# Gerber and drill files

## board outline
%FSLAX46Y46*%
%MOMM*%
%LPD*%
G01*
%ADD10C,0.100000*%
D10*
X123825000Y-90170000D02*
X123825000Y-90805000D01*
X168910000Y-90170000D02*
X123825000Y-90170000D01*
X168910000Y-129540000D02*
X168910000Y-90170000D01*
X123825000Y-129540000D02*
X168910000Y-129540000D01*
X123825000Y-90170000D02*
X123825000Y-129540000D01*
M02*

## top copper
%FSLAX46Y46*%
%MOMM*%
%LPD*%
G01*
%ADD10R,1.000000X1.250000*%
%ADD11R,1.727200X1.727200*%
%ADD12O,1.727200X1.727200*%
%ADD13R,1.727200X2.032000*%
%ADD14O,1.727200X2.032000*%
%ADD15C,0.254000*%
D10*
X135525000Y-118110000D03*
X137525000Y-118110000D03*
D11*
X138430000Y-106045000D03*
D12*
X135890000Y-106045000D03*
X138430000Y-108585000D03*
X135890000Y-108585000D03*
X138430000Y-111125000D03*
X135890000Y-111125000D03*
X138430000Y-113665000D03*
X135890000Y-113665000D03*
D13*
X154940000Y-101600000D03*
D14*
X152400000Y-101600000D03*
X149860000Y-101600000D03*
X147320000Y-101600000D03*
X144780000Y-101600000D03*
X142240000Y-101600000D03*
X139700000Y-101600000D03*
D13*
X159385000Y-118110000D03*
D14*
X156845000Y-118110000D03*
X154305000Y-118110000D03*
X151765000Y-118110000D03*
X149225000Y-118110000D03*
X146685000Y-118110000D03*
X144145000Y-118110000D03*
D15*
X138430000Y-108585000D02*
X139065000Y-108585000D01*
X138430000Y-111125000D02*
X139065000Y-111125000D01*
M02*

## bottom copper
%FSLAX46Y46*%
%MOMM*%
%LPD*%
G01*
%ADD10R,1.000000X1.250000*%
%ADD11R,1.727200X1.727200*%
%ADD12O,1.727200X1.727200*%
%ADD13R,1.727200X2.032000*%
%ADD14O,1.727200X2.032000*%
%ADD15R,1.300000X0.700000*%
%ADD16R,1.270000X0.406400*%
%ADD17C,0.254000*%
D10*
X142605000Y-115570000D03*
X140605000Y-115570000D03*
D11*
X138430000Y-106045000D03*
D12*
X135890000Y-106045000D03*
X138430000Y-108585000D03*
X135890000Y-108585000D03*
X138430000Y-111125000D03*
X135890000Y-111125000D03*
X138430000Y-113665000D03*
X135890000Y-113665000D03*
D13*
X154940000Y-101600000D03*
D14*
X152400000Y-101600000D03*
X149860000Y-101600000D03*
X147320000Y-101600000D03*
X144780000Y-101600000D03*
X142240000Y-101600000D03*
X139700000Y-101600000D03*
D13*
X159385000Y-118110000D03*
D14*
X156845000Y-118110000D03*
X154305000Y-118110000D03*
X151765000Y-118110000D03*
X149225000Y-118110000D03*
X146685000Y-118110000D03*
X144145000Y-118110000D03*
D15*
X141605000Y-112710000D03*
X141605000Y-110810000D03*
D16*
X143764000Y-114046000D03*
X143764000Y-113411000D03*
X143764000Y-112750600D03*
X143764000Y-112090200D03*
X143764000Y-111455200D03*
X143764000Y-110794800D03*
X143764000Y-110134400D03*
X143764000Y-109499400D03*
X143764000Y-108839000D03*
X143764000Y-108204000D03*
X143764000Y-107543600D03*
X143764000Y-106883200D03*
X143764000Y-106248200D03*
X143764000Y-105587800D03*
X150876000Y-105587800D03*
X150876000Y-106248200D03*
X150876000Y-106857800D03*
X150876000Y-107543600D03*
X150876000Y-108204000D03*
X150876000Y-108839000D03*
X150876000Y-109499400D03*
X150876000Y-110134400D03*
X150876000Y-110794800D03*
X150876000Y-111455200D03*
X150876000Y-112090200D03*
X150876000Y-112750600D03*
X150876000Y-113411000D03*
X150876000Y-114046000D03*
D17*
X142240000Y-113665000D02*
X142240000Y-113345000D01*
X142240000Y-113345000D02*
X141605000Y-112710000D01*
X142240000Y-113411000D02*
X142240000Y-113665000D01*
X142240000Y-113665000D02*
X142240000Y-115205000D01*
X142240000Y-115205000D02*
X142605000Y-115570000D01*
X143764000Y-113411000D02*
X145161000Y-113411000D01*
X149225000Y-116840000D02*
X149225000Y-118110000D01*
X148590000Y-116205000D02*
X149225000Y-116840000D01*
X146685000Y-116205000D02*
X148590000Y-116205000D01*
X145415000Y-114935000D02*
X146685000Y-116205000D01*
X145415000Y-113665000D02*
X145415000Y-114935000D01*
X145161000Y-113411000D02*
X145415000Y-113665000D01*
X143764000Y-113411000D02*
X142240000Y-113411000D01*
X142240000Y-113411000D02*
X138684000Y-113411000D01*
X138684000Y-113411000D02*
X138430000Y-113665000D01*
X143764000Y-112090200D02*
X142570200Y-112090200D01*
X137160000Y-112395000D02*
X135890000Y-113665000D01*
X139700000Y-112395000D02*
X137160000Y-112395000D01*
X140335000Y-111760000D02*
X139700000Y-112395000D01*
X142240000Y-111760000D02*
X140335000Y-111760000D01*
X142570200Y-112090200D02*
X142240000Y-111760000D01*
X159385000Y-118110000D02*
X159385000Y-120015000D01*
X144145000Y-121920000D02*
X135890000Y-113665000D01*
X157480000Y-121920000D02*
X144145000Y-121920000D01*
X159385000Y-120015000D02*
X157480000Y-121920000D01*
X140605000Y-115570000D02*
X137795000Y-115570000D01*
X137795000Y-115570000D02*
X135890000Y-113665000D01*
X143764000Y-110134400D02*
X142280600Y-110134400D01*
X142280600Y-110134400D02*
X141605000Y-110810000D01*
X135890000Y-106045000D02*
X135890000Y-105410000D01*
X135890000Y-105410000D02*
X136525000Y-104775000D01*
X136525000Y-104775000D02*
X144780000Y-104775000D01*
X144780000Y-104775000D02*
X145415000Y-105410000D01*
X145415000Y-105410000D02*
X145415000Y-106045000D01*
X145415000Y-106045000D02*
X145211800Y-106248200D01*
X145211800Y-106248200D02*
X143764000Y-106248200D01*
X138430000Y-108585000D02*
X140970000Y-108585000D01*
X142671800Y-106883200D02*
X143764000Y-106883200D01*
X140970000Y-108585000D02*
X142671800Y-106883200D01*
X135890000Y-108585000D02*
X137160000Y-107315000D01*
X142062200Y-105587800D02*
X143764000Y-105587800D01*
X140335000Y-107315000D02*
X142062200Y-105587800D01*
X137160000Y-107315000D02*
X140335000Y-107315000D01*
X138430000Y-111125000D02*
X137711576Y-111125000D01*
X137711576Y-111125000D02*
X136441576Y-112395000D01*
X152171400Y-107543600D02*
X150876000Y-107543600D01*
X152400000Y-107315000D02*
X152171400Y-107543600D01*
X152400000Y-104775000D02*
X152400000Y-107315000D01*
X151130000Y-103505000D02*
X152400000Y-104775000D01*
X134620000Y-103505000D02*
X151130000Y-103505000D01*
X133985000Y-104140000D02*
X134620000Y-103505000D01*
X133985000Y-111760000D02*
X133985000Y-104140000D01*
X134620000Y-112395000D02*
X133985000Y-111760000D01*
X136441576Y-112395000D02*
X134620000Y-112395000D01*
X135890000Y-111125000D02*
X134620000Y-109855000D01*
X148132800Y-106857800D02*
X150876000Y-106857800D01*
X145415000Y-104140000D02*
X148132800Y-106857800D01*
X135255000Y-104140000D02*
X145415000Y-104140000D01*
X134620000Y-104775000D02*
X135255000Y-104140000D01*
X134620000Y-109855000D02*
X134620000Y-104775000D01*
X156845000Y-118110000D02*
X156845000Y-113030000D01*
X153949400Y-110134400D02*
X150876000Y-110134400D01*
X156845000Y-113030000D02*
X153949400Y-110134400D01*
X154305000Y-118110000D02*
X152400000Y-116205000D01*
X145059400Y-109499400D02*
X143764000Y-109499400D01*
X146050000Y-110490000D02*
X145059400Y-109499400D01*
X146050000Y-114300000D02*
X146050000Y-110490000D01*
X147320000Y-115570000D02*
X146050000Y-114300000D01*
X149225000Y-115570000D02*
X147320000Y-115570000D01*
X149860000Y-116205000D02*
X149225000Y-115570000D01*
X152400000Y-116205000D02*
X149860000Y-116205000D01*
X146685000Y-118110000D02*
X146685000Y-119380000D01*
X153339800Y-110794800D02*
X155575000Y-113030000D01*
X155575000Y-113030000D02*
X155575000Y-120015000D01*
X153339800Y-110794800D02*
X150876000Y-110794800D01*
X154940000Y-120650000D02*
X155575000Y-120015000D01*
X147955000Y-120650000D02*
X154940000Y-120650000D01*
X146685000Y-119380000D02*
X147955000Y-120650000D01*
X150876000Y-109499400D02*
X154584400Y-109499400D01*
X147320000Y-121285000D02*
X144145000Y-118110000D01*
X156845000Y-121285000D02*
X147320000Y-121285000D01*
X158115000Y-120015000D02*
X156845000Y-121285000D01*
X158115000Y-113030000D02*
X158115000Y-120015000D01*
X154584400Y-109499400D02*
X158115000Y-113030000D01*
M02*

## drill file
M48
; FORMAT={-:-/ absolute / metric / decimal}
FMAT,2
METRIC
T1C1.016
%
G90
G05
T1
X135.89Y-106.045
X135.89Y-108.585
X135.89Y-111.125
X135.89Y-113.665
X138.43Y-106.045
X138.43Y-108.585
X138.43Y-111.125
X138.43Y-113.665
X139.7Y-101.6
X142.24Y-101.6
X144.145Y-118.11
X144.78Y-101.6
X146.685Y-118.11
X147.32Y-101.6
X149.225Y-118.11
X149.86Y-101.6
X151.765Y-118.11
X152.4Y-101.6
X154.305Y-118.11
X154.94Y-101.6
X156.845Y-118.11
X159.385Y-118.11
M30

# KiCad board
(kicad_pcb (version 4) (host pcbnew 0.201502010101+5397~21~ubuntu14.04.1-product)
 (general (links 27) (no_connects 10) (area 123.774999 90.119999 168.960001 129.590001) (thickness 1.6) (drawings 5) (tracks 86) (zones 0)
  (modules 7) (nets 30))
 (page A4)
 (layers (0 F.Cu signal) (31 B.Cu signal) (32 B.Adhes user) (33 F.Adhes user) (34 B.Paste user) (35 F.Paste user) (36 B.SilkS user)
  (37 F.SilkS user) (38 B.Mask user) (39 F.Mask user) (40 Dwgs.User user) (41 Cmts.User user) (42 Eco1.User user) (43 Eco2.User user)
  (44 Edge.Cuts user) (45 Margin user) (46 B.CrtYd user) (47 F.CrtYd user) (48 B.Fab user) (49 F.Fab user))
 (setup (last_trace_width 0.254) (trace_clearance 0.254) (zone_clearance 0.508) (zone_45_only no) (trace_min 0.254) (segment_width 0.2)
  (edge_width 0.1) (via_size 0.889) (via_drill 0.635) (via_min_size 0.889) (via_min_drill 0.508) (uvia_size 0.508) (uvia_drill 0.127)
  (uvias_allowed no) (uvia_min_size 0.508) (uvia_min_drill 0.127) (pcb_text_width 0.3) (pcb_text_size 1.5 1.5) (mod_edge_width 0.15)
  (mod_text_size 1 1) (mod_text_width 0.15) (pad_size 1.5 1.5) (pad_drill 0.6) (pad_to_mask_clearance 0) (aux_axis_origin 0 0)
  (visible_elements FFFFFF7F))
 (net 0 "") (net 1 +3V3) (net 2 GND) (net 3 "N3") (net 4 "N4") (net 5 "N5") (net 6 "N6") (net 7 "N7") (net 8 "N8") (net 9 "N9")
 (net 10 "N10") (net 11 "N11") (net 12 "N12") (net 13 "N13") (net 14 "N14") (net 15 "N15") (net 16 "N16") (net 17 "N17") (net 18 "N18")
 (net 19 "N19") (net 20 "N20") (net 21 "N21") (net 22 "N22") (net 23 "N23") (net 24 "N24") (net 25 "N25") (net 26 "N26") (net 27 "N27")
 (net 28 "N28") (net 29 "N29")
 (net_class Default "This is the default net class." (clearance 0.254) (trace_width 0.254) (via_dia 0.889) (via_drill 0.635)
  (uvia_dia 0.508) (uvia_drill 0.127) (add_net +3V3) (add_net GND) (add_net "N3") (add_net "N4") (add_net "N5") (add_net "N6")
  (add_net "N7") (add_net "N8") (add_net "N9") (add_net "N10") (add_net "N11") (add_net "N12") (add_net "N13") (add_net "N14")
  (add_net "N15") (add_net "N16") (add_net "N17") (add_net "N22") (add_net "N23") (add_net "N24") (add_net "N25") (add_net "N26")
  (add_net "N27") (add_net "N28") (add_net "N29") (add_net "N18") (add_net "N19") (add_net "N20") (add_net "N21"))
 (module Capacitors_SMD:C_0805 (layer B.Cu) (at 141.605 115.57 180)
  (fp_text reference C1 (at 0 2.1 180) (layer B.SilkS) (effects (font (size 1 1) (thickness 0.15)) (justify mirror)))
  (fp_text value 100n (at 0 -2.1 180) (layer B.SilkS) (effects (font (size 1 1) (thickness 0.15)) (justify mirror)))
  (pad 1 smd rect (at -1 0 180) (size 1 1.25) (layers B.Cu B.Paste B.Mask) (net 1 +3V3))
  (pad 2 smd rect (at 1 0 180) (size 1 1.25) (layers B.Cu B.Paste B.Mask) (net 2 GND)))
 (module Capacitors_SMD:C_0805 (layer F.Cu) (at 136.525 118.11)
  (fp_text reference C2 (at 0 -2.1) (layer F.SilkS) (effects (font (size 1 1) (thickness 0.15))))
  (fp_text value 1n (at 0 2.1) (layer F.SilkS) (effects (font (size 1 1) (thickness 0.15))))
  (pad 1 smd rect (at -1 0) (size 1 1.25) (layers F.Cu F.Paste F.Mask) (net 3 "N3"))
  (pad 2 smd rect (at 1 0) (size 1 1.25) (layers F.Cu F.Paste F.Mask) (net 2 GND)))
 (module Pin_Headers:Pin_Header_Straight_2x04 (layer B.Cu) (at 137.16 109.855 270)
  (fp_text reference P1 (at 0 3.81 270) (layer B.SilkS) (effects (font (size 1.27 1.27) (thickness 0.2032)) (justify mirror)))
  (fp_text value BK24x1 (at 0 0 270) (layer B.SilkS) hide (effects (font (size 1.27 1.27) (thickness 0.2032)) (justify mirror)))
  (pad 1 thru_hole rect (at -3.81 -1.27 270) (size 1.7272 1.7272) (drill 1.016) (layers *.Cu *.Mask B.SilkS) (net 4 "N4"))
  (pad 2 thru_hole oval (at -3.81 1.27 270) (size 1.7272 1.7272) (drill 1.016) (layers *.Cu *.Mask B.SilkS) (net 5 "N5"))
  (pad 3 thru_hole oval (at -1.27 -1.27 270) (size 1.7272 1.7272) (drill 1.016) (layers *.Cu *.Mask B.SilkS) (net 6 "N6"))
  (pad 4 thru_hole oval (at -1.27 1.27 270) (size 1.7272 1.7272) (drill 1.016) (layers *.Cu *.Mask B.SilkS) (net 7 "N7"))
  (pad 5 thru_hole oval (at 1.27 -1.27 270) (size 1.7272 1.7272) (drill 1.016) (layers *.Cu *.Mask B.SilkS) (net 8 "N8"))
  (pad 6 thru_hole oval (at 1.27 1.27 270) (size 1.7272 1.7272) (drill 1.016) (layers *.Cu *.Mask B.SilkS) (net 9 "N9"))
  (pad 7 thru_hole oval (at 3.81 -1.27 270) (size 1.7272 1.7272) (drill 1.016) (layers *.Cu *.Mask B.SilkS) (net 1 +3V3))
  (pad 8 thru_hole oval (at 3.81 1.27 270) (size 1.7272 1.7272) (drill 1.016) (layers *.Cu *.Mask B.SilkS) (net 2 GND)))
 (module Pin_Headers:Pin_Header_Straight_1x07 (layer B.Cu) (at 147.32 101.6 180)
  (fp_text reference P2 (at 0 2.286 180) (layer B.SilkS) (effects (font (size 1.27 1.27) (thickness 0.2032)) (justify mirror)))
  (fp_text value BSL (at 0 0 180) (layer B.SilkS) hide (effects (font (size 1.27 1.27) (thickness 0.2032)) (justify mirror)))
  (pad 1 thru_hole rect (at -7.62 0 180) (size 1.7272 2.032) (drill 1.016) (layers *.Cu *.Mask B.SilkS) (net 1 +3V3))
  (pad 2 thru_hole oval (at -5.08 0 180) (size 1.7272 2.032) (drill 1.016) (layers *.Cu *.Mask B.SilkS) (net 2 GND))
  (pad 3 thru_hole oval (at -2.54 0 180) (size 1.7272 2.032) (drill 1.016) (layers *.Cu *.Mask B.SilkS) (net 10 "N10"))
  (pad 4 thru_hole oval (at 0 0 180) (size 1.7272 2.032) (drill 1.016) (layers *.Cu *.Mask B.SilkS) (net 3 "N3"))
  (pad 5 thru_hole oval (at 2.54 0 180) (size 1.7272 2.032) (drill 1.016) (layers *.Cu *.Mask B.SilkS) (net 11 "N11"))
  (pad 6 thru_hole oval (at 5.08 0 180) (size 1.7272 2.032) (drill 1.016) (layers *.Cu *.Mask B.SilkS) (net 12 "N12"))
  (pad 7 thru_hole oval (at 7.62 0 180) (size 1.7272 2.032) (drill 1.016) (layers *.Cu *.Mask B.SilkS) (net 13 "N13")))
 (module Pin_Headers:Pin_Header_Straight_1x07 (layer B.Cu) (at 151.765 118.11 180)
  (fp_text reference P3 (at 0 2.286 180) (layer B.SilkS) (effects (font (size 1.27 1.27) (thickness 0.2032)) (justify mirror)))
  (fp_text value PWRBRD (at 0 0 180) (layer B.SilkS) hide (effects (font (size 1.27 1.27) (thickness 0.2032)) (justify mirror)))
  (pad 1 thru_hole rect (at -7.62 0 180) (size 1.7272 2.032) (drill 1.016) (layers *.Cu *.Mask B.SilkS) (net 2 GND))
  (pad 2 thru_hole oval (at -5.08 0 180) (size 1.7272 2.032) (drill 1.016) (layers *.Cu *.Mask B.SilkS) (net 11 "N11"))
  (pad 3 thru_hole oval (at -2.54 0 180) (size 1.7272 2.032) (drill 1.016) (layers *.Cu *.Mask B.SilkS) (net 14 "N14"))
  (pad 4 thru_hole oval (at 0 0 180) (size 1.7272 2.032) (drill 1.016) (layers *.Cu *.Mask B.SilkS) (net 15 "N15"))
  (pad 5 thru_hole oval (at 2.54 0 180) (size 1.7272 2.032) (drill 1.016) (layers *.Cu *.Mask B.SilkS) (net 1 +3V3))
  (pad 6 thru_hole oval (at 5.08 0 180) (size 1.7272 2.032) (drill 1.016) (layers *.Cu *.Mask B.SilkS) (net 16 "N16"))
  (pad 7 thru_hole oval (at 7.62 0 180) (size 1.7272 2.032) (drill 1.016) (layers *.Cu *.Mask B.SilkS) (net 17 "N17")))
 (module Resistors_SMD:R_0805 (layer B.Cu) (at 141.605 111.76 90)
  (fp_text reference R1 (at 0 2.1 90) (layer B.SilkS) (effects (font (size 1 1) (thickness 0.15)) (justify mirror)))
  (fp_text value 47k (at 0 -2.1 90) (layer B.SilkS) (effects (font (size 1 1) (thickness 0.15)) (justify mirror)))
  (pad 1 smd rect (at -0.95 0 90) (size 0.7 1.3) (layers B.Cu B.Paste B.Mask) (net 1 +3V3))
  (pad 2 smd rect (at 0.95 0 90) (size 0.7 1.3) (layers B.Cu B.Paste B.Mask) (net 3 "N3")))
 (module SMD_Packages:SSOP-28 (layer B.Cu) (at 147.32 109.855 90)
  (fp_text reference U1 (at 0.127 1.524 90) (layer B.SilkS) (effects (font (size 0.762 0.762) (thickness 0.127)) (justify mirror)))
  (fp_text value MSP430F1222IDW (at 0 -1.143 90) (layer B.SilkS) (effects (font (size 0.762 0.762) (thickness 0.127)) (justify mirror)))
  (pad 1 smd rect (at -4.191 -3.556 90) (size 0.4064 1.27) (layers B.Cu B.Paste B.Mask) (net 10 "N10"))
  (pad 2 smd rect (at -3.556 -3.556 90) (size 0.4064 1.27) (layers B.Cu B.Paste B.Mask) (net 1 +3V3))
  (pad 3 smd rect (at -2.8956 -3.556 90) (size 0.4064 1.27) (layers B.Cu B.Paste B.Mask) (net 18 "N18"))
  (pad 4 smd rect (at -2.2352 -3.556 90) (size 0.4064 1.27) (layers B.Cu B.Paste B.Mask) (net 2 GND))
  (pad 5 smd rect (at -1.6002 -3.556 90) (size 0.4064 1.27) (layers B.Cu B.Paste B.Mask) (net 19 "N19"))
  (pad 6 smd rect (at -0.9398 -3.556 90) (size 0.4064 1.27) (layers B.Cu B.Paste B.Mask) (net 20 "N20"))
  (pad 7 smd rect (at -0.2794 -3.556 90) (size 0.4064 1.27) (layers B.Cu B.Paste B.Mask) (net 3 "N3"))
  (pad 8 smd rect (at 0.3556 -3.556 90) (size 0.4064 1.27) (layers B.Cu B.Paste B.Mask) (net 14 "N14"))
  (pad 9 smd rect (at 1.016 -3.556 90) (size 0.4064 1.27) (layers B.Cu B.Paste B.Mask) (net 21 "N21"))
  (pad 10 smd rect (at 1.651 -3.556 90) (size 0.4064 1.27) (layers B.Cu B.Paste B.Mask) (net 12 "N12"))
  (pad 11 smd rect (at 2.3114 -3.556 90) (size 0.4064 1.27) (layers B.Cu B.Paste B.Mask) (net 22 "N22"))
  (pad 12 smd rect (at 2.9718 -3.556 90) (size 0.4064 1.27) (layers B.Cu B.Paste B.Mask) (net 6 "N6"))
  (pad 13 smd rect (at 3.6068 -3.556 90) (size 0.4064 1.27) (layers B.Cu B.Paste B.Mask) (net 5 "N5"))
  (pad 14 smd rect (at 4.2672 -3.556 90) (size 0.4064 1.27) (layers B.Cu B.Paste B.Mask) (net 7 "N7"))
  (pad 15 smd rect (at 4.2672 3.556 90) (size 0.4064 1.27) (layers B.Cu B.Paste B.Mask) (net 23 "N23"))
  (pad 16 smd rect (at 3.6068 3.556 90) (size 0.4064 1.27) (layers B.Cu B.Paste B.Mask) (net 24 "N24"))
  (pad 17 smd rect (at 2.9972 3.556 90) (size 0.4064 1.27) (layers B.Cu B.Paste B.Mask) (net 9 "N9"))
  (pad 18 smd rect (at 2.3114 3.556 90) (size 0.4064 1.27) (layers B.Cu B.Paste B.Mask) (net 8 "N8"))
  (pad 19 smd rect (at 1.651 3.556 90) (size 0.4064 1.27) (layers B.Cu B.Paste B.Mask) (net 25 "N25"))
  (pad 20 smd rect (at 1.016 3.556 90) (size 0.4064 1.27) (layers B.Cu B.Paste B.Mask) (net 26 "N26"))
  (pad 21 smd rect (at 0.3556 3.556 90) (size 0.4064 1.27) (layers B.Cu B.Paste B.Mask) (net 17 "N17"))
  (pad 22 smd rect (at -0.2794 3.556 90) (size 0.4064 1.27) (layers B.Cu B.Paste B.Mask) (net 11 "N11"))
  (pad 23 smd rect (at -0.9398 3.556 90) (size 0.4064 1.27) (layers B.Cu B.Paste B.Mask) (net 16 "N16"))
  (pad 24 smd rect (at -1.6002 3.556 90) (size 0.4064 1.27) (layers B.Cu B.Paste B.Mask) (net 15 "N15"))
  (pad 25 smd rect (at -2.2352 3.556 90) (size 0.4064 1.27) (layers B.Cu B.Paste B.Mask) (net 13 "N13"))
  (pad 26 smd rect (at -2.8956 3.556 90) (size 0.4064 1.27) (layers B.Cu B.Paste B.Mask) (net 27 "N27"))
  (pad 27 smd rect (at -3.556 3.556 90) (size 0.4064 1.27) (layers B.Cu B.Paste B.Mask) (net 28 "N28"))
  (pad 28 smd rect (at -4.191 3.556 90) (size 0.4064 1.27) (layers B.Cu B.Paste B.Mask) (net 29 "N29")))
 (gr_line (start 123.825 90.17) (end 123.825 90.805) (angle 90) (layer Edge.Cuts) (width 0.1))
 (gr_line (start 168.91 90.17) (end 123.825 90.17) (angle 90) (layer Edge.Cuts) (width 0.1))
 (gr_line (start 168.91 129.54) (end 168.91 90.17) (angle 90) (layer Edge.Cuts) (width 0.1))
 (gr_line (start 123.825 129.54) (end 168.91 129.54) (angle 90) (layer Edge.Cuts) (width 0.1))
 (gr_line (start 123.825 90.17) (end 123.825 129.54) (angle 90) (layer Edge.Cuts) (width 0.1))
 (segment (start 142.24 113.665) (end 142.24 113.345) (width 0.254) (layer B.Cu) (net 1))
 (segment (start 142.24 113.345) (end 141.605 112.71) (width 0.254) (layer B.Cu) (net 1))
 (segment (start 142.24 113.411) (end 142.24 113.665) (width 0.254) (layer B.Cu) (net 1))
 (segment (start 142.24 113.665) (end 142.24 115.205) (width 0.254) (layer B.Cu) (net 1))
 (segment (start 142.24 115.205) (end 142.605 115.57) (width 0.254) (layer B.Cu) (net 1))
 (segment (start 143.764 113.411) (end 145.161 113.411) (width 0.254) (layer B.Cu) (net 1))
 (segment (start 149.225 116.84) (end 149.225 118.11) (width 0.254) (layer B.Cu) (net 1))
 (segment (start 148.59 116.205) (end 149.225 116.84) (width 0.254) (layer B.Cu) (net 1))
 (segment (start 146.685 116.205) (end 148.59 116.205) (width 0.254) (layer B.Cu) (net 1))
 (segment (start 145.415 114.935) (end 146.685 116.205) (width 0.254) (layer B.Cu) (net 1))
 (segment (start 145.415 113.665) (end 145.415 114.935) (width 0.254) (layer B.Cu) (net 1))
 (segment (start 145.161 113.411) (end 145.415 113.665) (width 0.254) (layer B.Cu) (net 1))
 (segment (start 143.764 113.411) (end 142.24 113.411) (width 0.254) (layer B.Cu) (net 1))
 (segment (start 142.24 113.411) (end 138.684 113.411) (width 0.254) (layer B.Cu) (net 1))
 (segment (start 138.684 113.411) (end 138.43 113.665) (width 0.254) (layer B.Cu) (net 1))
 (segment (start 143.764 112.0902) (end 142.5702 112.0902) (width 0.254) (layer B.Cu) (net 2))
 (segment (start 137.16 112.395) (end 135.89 113.665) (width 0.254) (layer B.Cu) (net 2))
 (segment (start 139.7 112.395) (end 137.16 112.395) (width 0.254) (layer B.Cu) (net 2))
 (segment (start 140.335 111.76) (end 139.7 112.395) (width 0.254) (layer B.Cu) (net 2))
 (segment (start 142.24 111.76) (end 140.335 111.76) (width 0.254) (layer B.Cu) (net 2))
 (segment (start 142.5702 112.0902) (end 142.24 111.76) (width 0.254) (layer B.Cu) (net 2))
 (segment (start 159.385 118.11) (end 159.385 120.015) (width 0.254) (layer B.Cu) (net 2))
 (segment (start 144.145 121.92) (end 135.89 113.665) (width 0.254) (layer B.Cu) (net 2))
 (segment (start 157.48 121.92) (end 144.145 121.92) (width 0.254) (layer B.Cu) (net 2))
 (segment (start 159.385 120.015) (end 157.48 121.92) (width 0.254) (layer B.Cu) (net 2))
 (segment (start 140.605 115.57) (end 137.795 115.57) (width 0.254) (layer B.Cu) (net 2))
 (segment (start 137.795 115.57) (end 135.89 113.665) (width 0.254) (layer B.Cu) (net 2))
 (segment (start 143.764 110.1344) (end 142.2806 110.1344) (width 0.254) (layer B.Cu) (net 3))
 (segment (start 142.2806 110.1344) (end 141.605 110.81) (width 0.254) (layer B.Cu) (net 3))
 (segment (start 135.89 106.045) (end 135.89 105.41) (width 0.254) (layer B.Cu) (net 5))
 (segment (start 135.89 105.41) (end 136.525 104.775) (width 0.254) (layer B.Cu) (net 5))
 (segment (start 136.525 104.775) (end 144.78 104.775) (width 0.254) (layer B.Cu) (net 5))
 (segment (start 144.78 104.775) (end 145.415 105.41) (width 0.254) (layer B.Cu) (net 5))
 (segment (start 145.415 105.41) (end 145.415 106.045) (width 0.254) (layer B.Cu) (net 5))
 (segment (start 145.415 106.045) (end 145.2118 106.2482) (width 0.254) (layer B.Cu) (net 5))
 (segment (start 145.2118 106.2482) (end 143.764 106.2482) (width 0.254) (layer B.Cu) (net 5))
 (segment (start 138.43 108.585) (end 140.97 108.585) (width 0.254) (layer B.Cu) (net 6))
 (segment (start 142.6718 106.8832) (end 143.764 106.8832) (width 0.254) (layer B.Cu) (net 6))
 (segment (start 140.97 108.585) (end 142.6718 106.8832) (width 0.254) (layer B.Cu) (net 6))
 (segment (start 138.43 108.585) (end 139.065 108.585) (width 0.254) (layer F.Cu) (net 6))
 (segment (start 135.89 108.585) (end 137.16 107.315) (width 0.254) (layer B.Cu) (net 7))
 (segment (start 142.0622 105.5878) (end 143.764 105.5878) (width 0.254) (layer B.Cu) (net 7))
 (segment (start 140.335 107.315) (end 142.0622 105.5878) (width 0.254) (layer B.Cu) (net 7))
 (segment (start 137.16 107.315) (end 140.335 107.315) (width 0.254) (layer B.Cu) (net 7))
 (segment (start 138.43 111.125) (end 137.711576 111.125) (width 0.254) (layer B.Cu) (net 8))
 (segment (start 137.711576 111.125) (end 136.441576 112.395) (width 0.254) (layer B.Cu) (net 8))
 (segment (start 152.1714 107.5436) (end 150.876 107.5436) (width 0.254) (layer B.Cu) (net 8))
 (segment (start 152.4 107.315) (end 152.1714 107.5436) (width 0.254) (layer B.Cu) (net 8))
 (segment (start 152.4 104.775) (end 152.4 107.315) (width 0.254) (layer B.Cu) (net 8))
 (segment (start 151.13 103.505) (end 152.4 104.775) (width 0.254) (layer B.Cu) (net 8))
 (segment (start 134.62 103.505) (end 151.13 103.505) (width 0.254) (layer B.Cu) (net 8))
 (segment (start 133.985 104.14) (end 134.62 103.505) (width 0.254) (layer B.Cu) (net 8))
 (segment (start 133.985 111.76) (end 133.985 104.14) (width 0.254) (layer B.Cu) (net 8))
 (segment (start 134.62 112.395) (end 133.985 111.76) (width 0.254) (layer B.Cu) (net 8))
 (segment (start 136.441576 112.395) (end 134.62 112.395) (width 0.254) (layer B.Cu) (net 8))
 (segment (start 138.43 111.125) (end 139.065 111.125) (width 0.254) (layer F.Cu) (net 8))
 (segment (start 135.89 111.125) (end 134.62 109.855) (width 0.254) (layer B.Cu) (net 9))
 (segment (start 148.1328 106.8578) (end 150.876 106.8578) (width 0.254) (layer B.Cu) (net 9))
 (segment (start 145.415 104.14) (end 148.1328 106.8578) (width 0.254) (layer B.Cu) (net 9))
 (segment (start 135.255 104.14) (end 145.415 104.14) (width 0.254) (layer B.Cu) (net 9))
 (segment (start 134.62 104.775) (end 135.255 104.14) (width 0.254) (layer B.Cu) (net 9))
 (segment (start 134.62 109.855) (end 134.62 104.775) (width 0.254) (layer B.Cu) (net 9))
 (segment (start 156.845 118.11) (end 156.845 113.03) (width 0.254) (layer B.Cu) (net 11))
 (segment (start 153.9494 110.1344) (end 150.876 110.1344) (width 0.254) (layer B.Cu) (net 11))
 (segment (start 156.845 113.03) (end 153.9494 110.1344) (width 0.254) (layer B.Cu) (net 11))
 (segment (start 154.305 118.11) (end 152.4 116.205) (width 0.254) (layer B.Cu) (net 14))
 (segment (start 145.0594 109.4994) (end 143.764 109.4994) (width 0.254) (layer B.Cu) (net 14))
 (segment (start 146.05 110.49) (end 145.0594 109.4994) (width 0.254) (layer B.Cu) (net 14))
 (segment (start 146.05 114.3) (end 146.05 110.49) (width 0.254) (layer B.Cu) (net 14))
 (segment (start 147.32 115.57) (end 146.05 114.3) (width 0.254) (layer B.Cu) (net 14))
 (segment (start 149.225 115.57) (end 147.32 115.57) (width 0.254) (layer B.Cu) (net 14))
 (segment (start 149.86 116.205) (end 149.225 115.57) (width 0.254) (layer B.Cu) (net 14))
 (segment (start 152.4 116.205) (end 149.86 116.205) (width 0.254) (layer B.Cu) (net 14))
 (segment (start 146.685 118.11) (end 146.685 119.38) (width 0.254) (layer B.Cu) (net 16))
 (segment (start 153.3398 110.7948) (end 155.575 113.03) (width 0.254) (layer B.Cu) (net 16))
 (segment (start 155.575 113.03) (end 155.575 120.015) (width 0.254) (layer B.Cu) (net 16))
 (segment (start 153.3398 110.7948) (end 150.876 110.7948) (width 0.254) (layer B.Cu) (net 16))
 (segment (start 154.94 120.65) (end 155.575 120.015) (width 0.254) (layer B.Cu) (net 16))
 (segment (start 147.955 120.65) (end 154.94 120.65) (width 0.254) (layer B.Cu) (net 16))
 (segment (start 146.685 119.38) (end 147.955 120.65) (width 0.254) (layer B.Cu) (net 16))
 (segment (start 150.876 109.4994) (end 154.5844 109.4994) (width 0.254) (layer B.Cu) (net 17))
 (segment (start 147.32 121.285) (end 144.145 118.11) (width 0.254) (layer B.Cu) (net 17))
 (segment (start 156.845 121.285) (end 147.32 121.285) (width 0.254) (layer B.Cu) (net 17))
 (segment (start 158.115 120.015) (end 156.845 121.285) (width 0.254) (layer B.Cu) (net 17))
 (segment (start 158.115 113.03) (end 158.115 120.015) (width 0.254) (layer B.Cu) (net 17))
 (segment (start 154.5844 109.4994) (end 158.115 113.03) (width 0.254) (layer B.Cu) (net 17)))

